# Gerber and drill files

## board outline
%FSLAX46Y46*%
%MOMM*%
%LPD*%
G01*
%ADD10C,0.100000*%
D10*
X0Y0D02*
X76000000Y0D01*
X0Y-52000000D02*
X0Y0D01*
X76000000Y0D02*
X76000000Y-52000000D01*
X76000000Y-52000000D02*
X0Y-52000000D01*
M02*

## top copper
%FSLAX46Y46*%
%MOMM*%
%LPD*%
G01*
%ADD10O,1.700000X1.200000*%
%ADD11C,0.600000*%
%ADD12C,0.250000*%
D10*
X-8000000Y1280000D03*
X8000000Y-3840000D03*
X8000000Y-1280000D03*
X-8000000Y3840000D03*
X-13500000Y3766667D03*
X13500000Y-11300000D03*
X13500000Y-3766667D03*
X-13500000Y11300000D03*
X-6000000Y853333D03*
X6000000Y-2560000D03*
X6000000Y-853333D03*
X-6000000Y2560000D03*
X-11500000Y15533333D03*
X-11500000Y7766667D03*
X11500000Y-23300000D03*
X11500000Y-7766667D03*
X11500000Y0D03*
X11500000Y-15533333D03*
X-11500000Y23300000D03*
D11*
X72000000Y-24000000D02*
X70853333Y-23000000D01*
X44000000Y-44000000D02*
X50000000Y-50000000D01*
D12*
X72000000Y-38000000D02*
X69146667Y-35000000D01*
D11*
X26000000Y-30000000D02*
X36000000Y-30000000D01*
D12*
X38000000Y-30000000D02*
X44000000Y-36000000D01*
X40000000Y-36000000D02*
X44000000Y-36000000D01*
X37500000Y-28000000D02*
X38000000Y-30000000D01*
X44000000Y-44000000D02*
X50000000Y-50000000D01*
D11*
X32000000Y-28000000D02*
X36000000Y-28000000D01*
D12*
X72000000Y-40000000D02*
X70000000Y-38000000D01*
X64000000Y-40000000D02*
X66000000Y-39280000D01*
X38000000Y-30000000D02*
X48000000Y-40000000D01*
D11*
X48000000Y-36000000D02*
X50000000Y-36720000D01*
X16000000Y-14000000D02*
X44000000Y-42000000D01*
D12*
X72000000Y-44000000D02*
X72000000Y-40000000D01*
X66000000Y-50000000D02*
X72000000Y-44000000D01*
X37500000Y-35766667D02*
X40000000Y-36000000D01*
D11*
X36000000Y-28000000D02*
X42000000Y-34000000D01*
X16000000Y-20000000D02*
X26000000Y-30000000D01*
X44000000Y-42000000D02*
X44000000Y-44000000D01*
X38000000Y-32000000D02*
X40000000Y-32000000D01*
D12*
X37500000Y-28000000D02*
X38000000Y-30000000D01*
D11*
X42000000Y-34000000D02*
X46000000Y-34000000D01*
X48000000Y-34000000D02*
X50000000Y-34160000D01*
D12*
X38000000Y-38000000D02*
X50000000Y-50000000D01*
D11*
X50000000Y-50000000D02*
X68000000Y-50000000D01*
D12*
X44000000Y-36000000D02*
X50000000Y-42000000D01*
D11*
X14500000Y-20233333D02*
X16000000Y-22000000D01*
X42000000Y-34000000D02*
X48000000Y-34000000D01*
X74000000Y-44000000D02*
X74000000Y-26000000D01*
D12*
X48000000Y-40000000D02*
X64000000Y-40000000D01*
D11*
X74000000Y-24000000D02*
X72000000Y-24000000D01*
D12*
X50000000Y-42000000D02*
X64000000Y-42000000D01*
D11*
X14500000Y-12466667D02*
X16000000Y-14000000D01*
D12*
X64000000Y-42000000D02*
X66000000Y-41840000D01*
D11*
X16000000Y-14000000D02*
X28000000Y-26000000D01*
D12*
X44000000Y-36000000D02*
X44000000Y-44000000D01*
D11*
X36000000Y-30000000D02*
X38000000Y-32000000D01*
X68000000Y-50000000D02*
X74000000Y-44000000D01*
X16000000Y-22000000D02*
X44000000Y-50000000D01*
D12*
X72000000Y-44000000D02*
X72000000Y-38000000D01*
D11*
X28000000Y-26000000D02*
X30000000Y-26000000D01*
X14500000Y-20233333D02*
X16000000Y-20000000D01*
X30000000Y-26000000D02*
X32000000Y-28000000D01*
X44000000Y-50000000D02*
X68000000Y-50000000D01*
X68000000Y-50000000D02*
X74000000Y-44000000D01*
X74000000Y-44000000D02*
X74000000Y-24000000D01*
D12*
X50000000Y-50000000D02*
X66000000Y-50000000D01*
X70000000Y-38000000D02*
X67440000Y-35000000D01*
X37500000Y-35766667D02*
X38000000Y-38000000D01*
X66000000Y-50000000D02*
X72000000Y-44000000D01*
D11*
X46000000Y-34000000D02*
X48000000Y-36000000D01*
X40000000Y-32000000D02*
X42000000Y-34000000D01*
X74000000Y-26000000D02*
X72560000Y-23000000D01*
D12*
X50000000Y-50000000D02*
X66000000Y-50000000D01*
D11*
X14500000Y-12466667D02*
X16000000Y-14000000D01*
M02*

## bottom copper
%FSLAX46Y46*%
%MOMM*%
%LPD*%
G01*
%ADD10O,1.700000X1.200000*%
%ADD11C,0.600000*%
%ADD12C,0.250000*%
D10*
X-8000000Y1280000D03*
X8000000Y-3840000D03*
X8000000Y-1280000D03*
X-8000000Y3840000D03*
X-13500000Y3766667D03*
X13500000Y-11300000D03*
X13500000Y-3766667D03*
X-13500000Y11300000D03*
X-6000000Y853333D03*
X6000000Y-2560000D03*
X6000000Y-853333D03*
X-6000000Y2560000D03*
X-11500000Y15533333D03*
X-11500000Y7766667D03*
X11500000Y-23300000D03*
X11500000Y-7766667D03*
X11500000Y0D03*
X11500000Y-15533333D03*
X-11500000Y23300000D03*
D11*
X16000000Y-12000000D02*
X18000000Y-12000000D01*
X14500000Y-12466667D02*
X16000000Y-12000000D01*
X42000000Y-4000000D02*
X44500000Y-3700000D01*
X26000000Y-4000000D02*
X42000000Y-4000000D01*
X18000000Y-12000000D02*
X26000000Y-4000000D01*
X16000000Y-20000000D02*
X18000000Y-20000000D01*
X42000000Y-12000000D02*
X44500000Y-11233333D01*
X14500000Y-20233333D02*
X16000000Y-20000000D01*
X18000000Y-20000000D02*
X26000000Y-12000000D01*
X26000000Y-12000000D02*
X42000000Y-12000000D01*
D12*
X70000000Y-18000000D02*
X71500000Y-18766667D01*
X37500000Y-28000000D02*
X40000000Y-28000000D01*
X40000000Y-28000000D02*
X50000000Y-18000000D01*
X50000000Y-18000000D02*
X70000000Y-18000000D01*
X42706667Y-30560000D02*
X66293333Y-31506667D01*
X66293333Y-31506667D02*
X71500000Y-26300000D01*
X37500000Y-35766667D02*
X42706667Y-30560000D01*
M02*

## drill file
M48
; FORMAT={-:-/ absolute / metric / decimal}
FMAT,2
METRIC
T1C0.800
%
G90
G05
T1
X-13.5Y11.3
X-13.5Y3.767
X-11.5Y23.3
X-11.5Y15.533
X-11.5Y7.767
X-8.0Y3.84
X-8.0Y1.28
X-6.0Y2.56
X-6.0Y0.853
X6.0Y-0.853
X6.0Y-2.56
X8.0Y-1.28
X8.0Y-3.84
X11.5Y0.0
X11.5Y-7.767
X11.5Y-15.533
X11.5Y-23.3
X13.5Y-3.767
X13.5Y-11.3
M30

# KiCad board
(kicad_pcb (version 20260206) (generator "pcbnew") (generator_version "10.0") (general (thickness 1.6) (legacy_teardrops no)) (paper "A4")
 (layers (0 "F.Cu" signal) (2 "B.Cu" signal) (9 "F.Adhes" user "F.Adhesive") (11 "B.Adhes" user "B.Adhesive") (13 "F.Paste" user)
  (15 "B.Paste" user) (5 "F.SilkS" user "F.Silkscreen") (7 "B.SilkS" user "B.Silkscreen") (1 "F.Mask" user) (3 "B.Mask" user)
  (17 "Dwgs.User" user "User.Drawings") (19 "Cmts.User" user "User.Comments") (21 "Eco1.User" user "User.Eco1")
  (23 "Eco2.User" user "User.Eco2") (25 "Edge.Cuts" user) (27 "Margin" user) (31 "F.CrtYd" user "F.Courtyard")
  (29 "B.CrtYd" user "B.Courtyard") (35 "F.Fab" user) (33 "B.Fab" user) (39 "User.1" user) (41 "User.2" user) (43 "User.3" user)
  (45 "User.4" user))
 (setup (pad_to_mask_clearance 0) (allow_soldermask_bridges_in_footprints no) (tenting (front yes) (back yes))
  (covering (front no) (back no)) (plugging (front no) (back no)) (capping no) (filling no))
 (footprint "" (layer "F.Cu") (at 58 38)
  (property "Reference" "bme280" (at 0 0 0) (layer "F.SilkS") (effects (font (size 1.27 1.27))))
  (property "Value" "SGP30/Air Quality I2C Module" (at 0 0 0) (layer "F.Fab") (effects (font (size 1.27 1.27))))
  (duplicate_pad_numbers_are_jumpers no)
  (pad "GND" thru_hole oval (at -66 -39.28) (size 1.7 1.2) (drill 0.8) (layers "*.Cu") (remove_unused_layers no) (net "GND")
   (thermal_bridge_angle 45))
  (pad "SCL" thru_hole oval (at -50 -34.16) (size 1.7 1.2) (drill 0.8) (layers "*.Cu") (remove_unused_layers no) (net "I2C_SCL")
   (thermal_bridge_angle 45))
  (pad "SDA" thru_hole oval (at -50 -36.72) (size 1.7 1.2) (drill 0.8) (layers "*.Cu") (remove_unused_layers no) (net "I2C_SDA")
   (thermal_bridge_angle 45))
  (pad "VCC" thru_hole oval (at -66 -41.84) (size 1.7 1.2) (drill 0.8) (layers "*.Cu") (remove_unused_layers no) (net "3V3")
   (thermal_bridge_angle 45)))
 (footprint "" (layer "F.Cu") (at 58 15)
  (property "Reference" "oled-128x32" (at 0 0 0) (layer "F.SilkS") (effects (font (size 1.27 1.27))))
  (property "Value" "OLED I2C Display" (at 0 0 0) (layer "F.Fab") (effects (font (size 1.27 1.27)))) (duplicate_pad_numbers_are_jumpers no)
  (pad "GND" thru_hole oval (at -71.5 -18.766667) (size 1.7 1.2) (drill 0.8) (layers "*.Cu") (remove_unused_layers no) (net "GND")
   (thermal_bridge_angle 45))
  (pad "SCL" thru_hole oval (at -44.5 -3.7) (size 1.7 1.2) (drill 0.8) (layers "*.Cu") (remove_unused_layers no) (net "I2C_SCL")
   (thermal_bridge_angle 45))
  (pad "SDA" thru_hole oval (at -44.5 -11.233333) (size 1.7 1.2) (drill 0.8) (layers "*.Cu") (remove_unused_layers no) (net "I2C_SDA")
   (thermal_bridge_angle 45))
  (pad "VCC" thru_hole oval (at -71.5 -26.3) (size 1.7 1.2) (drill 0.8) (layers "*.Cu") (remove_unused_layers no) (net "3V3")
   (thermal_bridge_angle 45)))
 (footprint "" (layer "F.Cu") (at 70 29 90)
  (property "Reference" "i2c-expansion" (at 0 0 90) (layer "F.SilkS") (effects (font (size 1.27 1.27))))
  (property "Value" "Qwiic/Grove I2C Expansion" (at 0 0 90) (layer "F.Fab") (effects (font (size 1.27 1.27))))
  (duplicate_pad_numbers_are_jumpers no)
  (pad "GND" thru_hole oval (at 29.853333 -76) (size 1.7 1.2) (drill 0.8) (layers "*.Cu") (remove_unused_layers no) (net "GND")
   (thermal_bridge_angle 45))
  (pad "SCL" thru_hole oval (at 26.44 -64) (size 1.7 1.2) (drill 0.8) (layers "*.Cu") (remove_unused_layers no) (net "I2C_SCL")
   (thermal_bridge_angle 45))
  (pad "SDA" thru_hole oval (at 28.146667 -64) (size 1.7 1.2) (drill 0.8) (layers "*.Cu") (remove_unused_layers no) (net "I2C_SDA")
   (thermal_bridge_angle 45))
  (pad "VCC" thru_hole oval (at 31.56 -76) (size 1.7 1.2) (drill 0.8) (layers "*.Cu") (remove_unused_layers no) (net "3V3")
   (thermal_bridge_angle 45)))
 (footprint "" (layer "F.Cu") (at 26 28)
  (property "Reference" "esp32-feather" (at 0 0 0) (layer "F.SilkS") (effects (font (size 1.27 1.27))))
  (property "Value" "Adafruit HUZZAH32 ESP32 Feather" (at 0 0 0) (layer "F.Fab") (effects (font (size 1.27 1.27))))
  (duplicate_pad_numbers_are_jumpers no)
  (pad "3V3" thru_hole oval (at -37.5 -43.533333) (size 1.7 1.2) (drill 0.8) (layers "*.Cu") (remove_unused_layers no) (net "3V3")
   (thermal_bridge_angle 45))
  (pad "GND" thru_hole oval (at -37.5 -35.766667) (size 1.7 1.2) (drill 0.8) (layers "*.Cu") (remove_unused_layers no) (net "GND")
   (thermal_bridge_angle 45))
  (pad "RX" thru_hole oval (at -14.5 -4.7) (size 1.7 1.2) (drill 0.8) (layers "*.Cu") (remove_unused_layers no) (thermal_bridge_angle 45))
  (pad "SCL" thru_hole oval (at -14.5 -20.233333) (size 1.7 1.2) (drill 0.8) (layers "*.Cu") (remove_unused_layers no) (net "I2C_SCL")
   (thermal_bridge_angle 45))
  (pad "SDA" thru_hole oval (at -14.5 -28) (size 1.7 1.2) (drill 0.8) (layers "*.Cu") (remove_unused_layers no) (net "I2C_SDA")
   (thermal_bridge_angle 45))
  (pad "TX" thru_hole oval (at -14.5 -12.466667) (size 1.7 1.2) (drill 0.8) (layers "*.Cu") (remove_unused_layers no)
   (thermal_bridge_angle 45))
  (pad "VIN" thru_hole oval (at -37.5 -51.3) (size 1.7 1.2) (drill 0.8) (layers "*.Cu") (remove_unused_layers no) (thermal_bridge_angle 45)))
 (gr_line (start 0 0) (end 76 0) (stroke (width 0.1) (type default)) (layer "Edge.Cuts"))
 (gr_line (start 0 52) (end 0 0) (stroke (width 0.1) (type default)) (layer "Edge.Cuts"))
 (gr_line (start 76 0) (end 76 52) (stroke (width 0.1) (type default)) (layer "Edge.Cuts"))
 (gr_line (start 76 52) (end 0 52) (stroke (width 0.1) (type default)) (layer "Edge.Cuts"))
 (segment (start 72 24) (end 70.853333 23) (width 0.6) (layer "F.Cu") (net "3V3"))
 (segment (start 44 44) (end 50 50) (width 0.6) (layer "F.Cu") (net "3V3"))
 (segment (start 72 38) (end 69.146667 35) (width 0.25) (layer "F.Cu") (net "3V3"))
 (segment (start 26 30) (end 36 30) (width 0.6) (layer "F.Cu") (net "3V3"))
 (segment (start 38 30) (end 44 36) (width 0.25) (layer "F.Cu") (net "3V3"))
 (segment (start 40 36) (end 44 36) (width 0.25) (layer "F.Cu") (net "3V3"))
 (segment (start 37.5 28) (end 38 30) (width 0.25) (layer "F.Cu") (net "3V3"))
 (segment (start 44 44) (end 50 50) (width 0.25) (layer "F.Cu") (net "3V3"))
 (segment (start 32 28) (end 36 28) (width 0.6) (layer "F.Cu") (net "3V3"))
 (segment (start 72 40) (end 70 38) (width 0.25) (layer "F.Cu") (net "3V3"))
 (segment (start 64 40) (end 66 39.28) (width 0.25) (layer "F.Cu") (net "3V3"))
 (segment (start 38 30) (end 48 40) (width 0.25) (layer "F.Cu") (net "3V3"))
 (segment (start 48 36) (end 50 36.72) (width 0.6) (layer "F.Cu") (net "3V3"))
 (segment (start 16 14) (end 44 42) (width 0.6) (layer "F.Cu") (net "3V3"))
 (segment (start 72 44) (end 72 40) (width 0.25) (layer "F.Cu") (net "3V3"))
 (segment (start 66 50) (end 72 44) (width 0.25) (layer "F.Cu") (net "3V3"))
 (segment (start 37.5 35.766667) (end 40 36) (width 0.25) (layer "F.Cu") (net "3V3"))
 (segment (start 36 28) (end 42 34) (width 0.6) (layer "F.Cu") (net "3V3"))
 (segment (start 16 20) (end 26 30) (width 0.6) (layer "F.Cu") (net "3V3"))
 (segment (start 44 42) (end 44 44) (width 0.6) (layer "F.Cu") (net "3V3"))
 (segment (start 38 32) (end 40 32) (width 0.6) (layer "F.Cu") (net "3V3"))
 (segment (start 37.5 28) (end 38 30) (width 0.25) (layer "F.Cu") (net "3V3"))
 (segment (start 42 34) (end 46 34) (width 0.6) (layer "F.Cu") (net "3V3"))
 (segment (start 48 34) (end 50 34.16) (width 0.6) (layer "F.Cu") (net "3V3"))
 (segment (start 38 38) (end 50 50) (width 0.25) (layer "F.Cu") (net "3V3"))
 (segment (start 50 50) (end 68 50) (width 0.6) (layer "F.Cu") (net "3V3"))
 (segment (start 44 36) (end 50 42) (width 0.25) (layer "F.Cu") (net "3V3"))
 (segment (start 14.5 20.233333) (end 16 22) (width 0.6) (layer "F.Cu") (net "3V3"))
 (segment (start 42 34) (end 48 34) (width 0.6) (layer "F.Cu") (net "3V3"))
 (segment (start 74 44) (end 74 26) (width 0.6) (layer "F.Cu") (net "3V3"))
 (segment (start 48 40) (end 64 40) (width 0.25) (layer "F.Cu") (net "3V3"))
 (segment (start 74 24) (end 72 24) (width 0.6) (layer "F.Cu") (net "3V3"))
 (segment (start 50 42) (end 64 42) (width 0.25) (layer "F.Cu") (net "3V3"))
 (segment (start 14.5 12.466667) (end 16 14) (width 0.6) (layer "F.Cu") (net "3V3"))
 (segment (start 64 42) (end 66 41.84) (width 0.25) (layer "F.Cu") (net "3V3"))
 (segment (start 16 14) (end 28 26) (width 0.6) (layer "F.Cu") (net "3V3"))
 (segment (start 44 36) (end 44 44) (width 0.25) (layer "F.Cu") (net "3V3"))
 (segment (start 36 30) (end 38 32) (width 0.6) (layer "F.Cu") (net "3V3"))
 (segment (start 68 50) (end 74 44) (width 0.6) (layer "F.Cu") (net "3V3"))
 (segment (start 16 22) (end 44 50) (width 0.6) (layer "F.Cu") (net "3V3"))
 (segment (start 72 44) (end 72 38) (width 0.25) (layer "F.Cu") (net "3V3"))
 (segment (start 28 26) (end 30 26) (width 0.6) (layer "F.Cu") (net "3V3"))
 (segment (start 14.5 20.233333) (end 16 20) (width 0.6) (layer "F.Cu") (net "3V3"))
 (segment (start 30 26) (end 32 28) (width 0.6) (layer "F.Cu") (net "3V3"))
 (segment (start 44 50) (end 68 50) (width 0.6) (layer "F.Cu") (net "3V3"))
 (segment (start 68 50) (end 74 44) (width 0.6) (layer "F.Cu") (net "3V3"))
 (segment (start 74 44) (end 74 24) (width 0.6) (layer "F.Cu") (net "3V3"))
 (segment (start 50 50) (end 66 50) (width 0.25) (layer "F.Cu") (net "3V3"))
 (segment (start 70 38) (end 67.44 35) (width 0.25) (layer "F.Cu") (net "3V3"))
 (segment (start 37.5 35.766667) (end 38 38) (width 0.25) (layer "F.Cu") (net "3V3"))
 (segment (start 66 50) (end 72 44) (width 0.25) (layer "F.Cu") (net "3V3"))
 (segment (start 46 34) (end 48 36) (width 0.6) (layer "F.Cu") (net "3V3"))
 (segment (start 40 32) (end 42 34) (width 0.6) (layer "F.Cu") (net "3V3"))
 (segment (start 74 26) (end 72.56 23) (width 0.6) (layer "F.Cu") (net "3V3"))
 (segment (start 50 50) (end 66 50) (width 0.25) (layer "F.Cu") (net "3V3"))
 (segment (start 14.5 12.466667) (end 16 14) (width 0.6) (layer "F.Cu") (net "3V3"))
 (segment (start 16 12) (end 18 12) (width 0.6) (layer "B.Cu") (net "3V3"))
 (segment (start 14.5 12.466667) (end 16 12) (width 0.6) (layer "B.Cu") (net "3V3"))
 (segment (start 42 4) (end 44.5 3.7) (width 0.6) (layer "B.Cu") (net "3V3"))
 (segment (start 26 4) (end 42 4) (width 0.6) (layer "B.Cu") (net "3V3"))
 (segment (start 18 12) (end 26 4) (width 0.6) (layer "B.Cu") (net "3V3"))
 (segment (start 16 20) (end 18 20) (width 0.6) (layer "B.Cu") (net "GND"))
 (segment (start 42 12) (end 44.5 11.233333) (width 0.6) (layer "B.Cu") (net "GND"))
 (segment (start 14.5 20.233333) (end 16 20) (width 0.6) (layer "B.Cu") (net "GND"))
 (segment (start 18 20) (end 26 12) (width 0.6) (layer "B.Cu") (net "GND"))
 (segment (start 26 12) (end 42 12) (width 0.6) (layer "B.Cu") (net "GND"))
 (segment (start 70 18) (end 71.5 18.766667) (width 0.25) (layer "B.Cu") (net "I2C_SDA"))
 (segment (start 37.5 28) (end 40 28) (width 0.25) (layer "B.Cu") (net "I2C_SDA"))
 (segment (start 40 28) (end 50 18) (width 0.25) (layer "B.Cu") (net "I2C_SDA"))
 (segment (start 50 18) (end 70 18) (width 0.25) (layer "B.Cu") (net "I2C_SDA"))
 (segment (start 42.706667 30.56) (end 66.293333 31.506667) (width 0.25) (layer "B.Cu") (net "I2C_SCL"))
 (segment (start 66.293333 31.506667) (end 71.5 26.3) (width 0.25) (layer "B.Cu") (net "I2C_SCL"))
 (segment (start 37.5 35.766667) (end 42.706667 30.56) (width 0.25) (layer "B.Cu") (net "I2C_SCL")))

